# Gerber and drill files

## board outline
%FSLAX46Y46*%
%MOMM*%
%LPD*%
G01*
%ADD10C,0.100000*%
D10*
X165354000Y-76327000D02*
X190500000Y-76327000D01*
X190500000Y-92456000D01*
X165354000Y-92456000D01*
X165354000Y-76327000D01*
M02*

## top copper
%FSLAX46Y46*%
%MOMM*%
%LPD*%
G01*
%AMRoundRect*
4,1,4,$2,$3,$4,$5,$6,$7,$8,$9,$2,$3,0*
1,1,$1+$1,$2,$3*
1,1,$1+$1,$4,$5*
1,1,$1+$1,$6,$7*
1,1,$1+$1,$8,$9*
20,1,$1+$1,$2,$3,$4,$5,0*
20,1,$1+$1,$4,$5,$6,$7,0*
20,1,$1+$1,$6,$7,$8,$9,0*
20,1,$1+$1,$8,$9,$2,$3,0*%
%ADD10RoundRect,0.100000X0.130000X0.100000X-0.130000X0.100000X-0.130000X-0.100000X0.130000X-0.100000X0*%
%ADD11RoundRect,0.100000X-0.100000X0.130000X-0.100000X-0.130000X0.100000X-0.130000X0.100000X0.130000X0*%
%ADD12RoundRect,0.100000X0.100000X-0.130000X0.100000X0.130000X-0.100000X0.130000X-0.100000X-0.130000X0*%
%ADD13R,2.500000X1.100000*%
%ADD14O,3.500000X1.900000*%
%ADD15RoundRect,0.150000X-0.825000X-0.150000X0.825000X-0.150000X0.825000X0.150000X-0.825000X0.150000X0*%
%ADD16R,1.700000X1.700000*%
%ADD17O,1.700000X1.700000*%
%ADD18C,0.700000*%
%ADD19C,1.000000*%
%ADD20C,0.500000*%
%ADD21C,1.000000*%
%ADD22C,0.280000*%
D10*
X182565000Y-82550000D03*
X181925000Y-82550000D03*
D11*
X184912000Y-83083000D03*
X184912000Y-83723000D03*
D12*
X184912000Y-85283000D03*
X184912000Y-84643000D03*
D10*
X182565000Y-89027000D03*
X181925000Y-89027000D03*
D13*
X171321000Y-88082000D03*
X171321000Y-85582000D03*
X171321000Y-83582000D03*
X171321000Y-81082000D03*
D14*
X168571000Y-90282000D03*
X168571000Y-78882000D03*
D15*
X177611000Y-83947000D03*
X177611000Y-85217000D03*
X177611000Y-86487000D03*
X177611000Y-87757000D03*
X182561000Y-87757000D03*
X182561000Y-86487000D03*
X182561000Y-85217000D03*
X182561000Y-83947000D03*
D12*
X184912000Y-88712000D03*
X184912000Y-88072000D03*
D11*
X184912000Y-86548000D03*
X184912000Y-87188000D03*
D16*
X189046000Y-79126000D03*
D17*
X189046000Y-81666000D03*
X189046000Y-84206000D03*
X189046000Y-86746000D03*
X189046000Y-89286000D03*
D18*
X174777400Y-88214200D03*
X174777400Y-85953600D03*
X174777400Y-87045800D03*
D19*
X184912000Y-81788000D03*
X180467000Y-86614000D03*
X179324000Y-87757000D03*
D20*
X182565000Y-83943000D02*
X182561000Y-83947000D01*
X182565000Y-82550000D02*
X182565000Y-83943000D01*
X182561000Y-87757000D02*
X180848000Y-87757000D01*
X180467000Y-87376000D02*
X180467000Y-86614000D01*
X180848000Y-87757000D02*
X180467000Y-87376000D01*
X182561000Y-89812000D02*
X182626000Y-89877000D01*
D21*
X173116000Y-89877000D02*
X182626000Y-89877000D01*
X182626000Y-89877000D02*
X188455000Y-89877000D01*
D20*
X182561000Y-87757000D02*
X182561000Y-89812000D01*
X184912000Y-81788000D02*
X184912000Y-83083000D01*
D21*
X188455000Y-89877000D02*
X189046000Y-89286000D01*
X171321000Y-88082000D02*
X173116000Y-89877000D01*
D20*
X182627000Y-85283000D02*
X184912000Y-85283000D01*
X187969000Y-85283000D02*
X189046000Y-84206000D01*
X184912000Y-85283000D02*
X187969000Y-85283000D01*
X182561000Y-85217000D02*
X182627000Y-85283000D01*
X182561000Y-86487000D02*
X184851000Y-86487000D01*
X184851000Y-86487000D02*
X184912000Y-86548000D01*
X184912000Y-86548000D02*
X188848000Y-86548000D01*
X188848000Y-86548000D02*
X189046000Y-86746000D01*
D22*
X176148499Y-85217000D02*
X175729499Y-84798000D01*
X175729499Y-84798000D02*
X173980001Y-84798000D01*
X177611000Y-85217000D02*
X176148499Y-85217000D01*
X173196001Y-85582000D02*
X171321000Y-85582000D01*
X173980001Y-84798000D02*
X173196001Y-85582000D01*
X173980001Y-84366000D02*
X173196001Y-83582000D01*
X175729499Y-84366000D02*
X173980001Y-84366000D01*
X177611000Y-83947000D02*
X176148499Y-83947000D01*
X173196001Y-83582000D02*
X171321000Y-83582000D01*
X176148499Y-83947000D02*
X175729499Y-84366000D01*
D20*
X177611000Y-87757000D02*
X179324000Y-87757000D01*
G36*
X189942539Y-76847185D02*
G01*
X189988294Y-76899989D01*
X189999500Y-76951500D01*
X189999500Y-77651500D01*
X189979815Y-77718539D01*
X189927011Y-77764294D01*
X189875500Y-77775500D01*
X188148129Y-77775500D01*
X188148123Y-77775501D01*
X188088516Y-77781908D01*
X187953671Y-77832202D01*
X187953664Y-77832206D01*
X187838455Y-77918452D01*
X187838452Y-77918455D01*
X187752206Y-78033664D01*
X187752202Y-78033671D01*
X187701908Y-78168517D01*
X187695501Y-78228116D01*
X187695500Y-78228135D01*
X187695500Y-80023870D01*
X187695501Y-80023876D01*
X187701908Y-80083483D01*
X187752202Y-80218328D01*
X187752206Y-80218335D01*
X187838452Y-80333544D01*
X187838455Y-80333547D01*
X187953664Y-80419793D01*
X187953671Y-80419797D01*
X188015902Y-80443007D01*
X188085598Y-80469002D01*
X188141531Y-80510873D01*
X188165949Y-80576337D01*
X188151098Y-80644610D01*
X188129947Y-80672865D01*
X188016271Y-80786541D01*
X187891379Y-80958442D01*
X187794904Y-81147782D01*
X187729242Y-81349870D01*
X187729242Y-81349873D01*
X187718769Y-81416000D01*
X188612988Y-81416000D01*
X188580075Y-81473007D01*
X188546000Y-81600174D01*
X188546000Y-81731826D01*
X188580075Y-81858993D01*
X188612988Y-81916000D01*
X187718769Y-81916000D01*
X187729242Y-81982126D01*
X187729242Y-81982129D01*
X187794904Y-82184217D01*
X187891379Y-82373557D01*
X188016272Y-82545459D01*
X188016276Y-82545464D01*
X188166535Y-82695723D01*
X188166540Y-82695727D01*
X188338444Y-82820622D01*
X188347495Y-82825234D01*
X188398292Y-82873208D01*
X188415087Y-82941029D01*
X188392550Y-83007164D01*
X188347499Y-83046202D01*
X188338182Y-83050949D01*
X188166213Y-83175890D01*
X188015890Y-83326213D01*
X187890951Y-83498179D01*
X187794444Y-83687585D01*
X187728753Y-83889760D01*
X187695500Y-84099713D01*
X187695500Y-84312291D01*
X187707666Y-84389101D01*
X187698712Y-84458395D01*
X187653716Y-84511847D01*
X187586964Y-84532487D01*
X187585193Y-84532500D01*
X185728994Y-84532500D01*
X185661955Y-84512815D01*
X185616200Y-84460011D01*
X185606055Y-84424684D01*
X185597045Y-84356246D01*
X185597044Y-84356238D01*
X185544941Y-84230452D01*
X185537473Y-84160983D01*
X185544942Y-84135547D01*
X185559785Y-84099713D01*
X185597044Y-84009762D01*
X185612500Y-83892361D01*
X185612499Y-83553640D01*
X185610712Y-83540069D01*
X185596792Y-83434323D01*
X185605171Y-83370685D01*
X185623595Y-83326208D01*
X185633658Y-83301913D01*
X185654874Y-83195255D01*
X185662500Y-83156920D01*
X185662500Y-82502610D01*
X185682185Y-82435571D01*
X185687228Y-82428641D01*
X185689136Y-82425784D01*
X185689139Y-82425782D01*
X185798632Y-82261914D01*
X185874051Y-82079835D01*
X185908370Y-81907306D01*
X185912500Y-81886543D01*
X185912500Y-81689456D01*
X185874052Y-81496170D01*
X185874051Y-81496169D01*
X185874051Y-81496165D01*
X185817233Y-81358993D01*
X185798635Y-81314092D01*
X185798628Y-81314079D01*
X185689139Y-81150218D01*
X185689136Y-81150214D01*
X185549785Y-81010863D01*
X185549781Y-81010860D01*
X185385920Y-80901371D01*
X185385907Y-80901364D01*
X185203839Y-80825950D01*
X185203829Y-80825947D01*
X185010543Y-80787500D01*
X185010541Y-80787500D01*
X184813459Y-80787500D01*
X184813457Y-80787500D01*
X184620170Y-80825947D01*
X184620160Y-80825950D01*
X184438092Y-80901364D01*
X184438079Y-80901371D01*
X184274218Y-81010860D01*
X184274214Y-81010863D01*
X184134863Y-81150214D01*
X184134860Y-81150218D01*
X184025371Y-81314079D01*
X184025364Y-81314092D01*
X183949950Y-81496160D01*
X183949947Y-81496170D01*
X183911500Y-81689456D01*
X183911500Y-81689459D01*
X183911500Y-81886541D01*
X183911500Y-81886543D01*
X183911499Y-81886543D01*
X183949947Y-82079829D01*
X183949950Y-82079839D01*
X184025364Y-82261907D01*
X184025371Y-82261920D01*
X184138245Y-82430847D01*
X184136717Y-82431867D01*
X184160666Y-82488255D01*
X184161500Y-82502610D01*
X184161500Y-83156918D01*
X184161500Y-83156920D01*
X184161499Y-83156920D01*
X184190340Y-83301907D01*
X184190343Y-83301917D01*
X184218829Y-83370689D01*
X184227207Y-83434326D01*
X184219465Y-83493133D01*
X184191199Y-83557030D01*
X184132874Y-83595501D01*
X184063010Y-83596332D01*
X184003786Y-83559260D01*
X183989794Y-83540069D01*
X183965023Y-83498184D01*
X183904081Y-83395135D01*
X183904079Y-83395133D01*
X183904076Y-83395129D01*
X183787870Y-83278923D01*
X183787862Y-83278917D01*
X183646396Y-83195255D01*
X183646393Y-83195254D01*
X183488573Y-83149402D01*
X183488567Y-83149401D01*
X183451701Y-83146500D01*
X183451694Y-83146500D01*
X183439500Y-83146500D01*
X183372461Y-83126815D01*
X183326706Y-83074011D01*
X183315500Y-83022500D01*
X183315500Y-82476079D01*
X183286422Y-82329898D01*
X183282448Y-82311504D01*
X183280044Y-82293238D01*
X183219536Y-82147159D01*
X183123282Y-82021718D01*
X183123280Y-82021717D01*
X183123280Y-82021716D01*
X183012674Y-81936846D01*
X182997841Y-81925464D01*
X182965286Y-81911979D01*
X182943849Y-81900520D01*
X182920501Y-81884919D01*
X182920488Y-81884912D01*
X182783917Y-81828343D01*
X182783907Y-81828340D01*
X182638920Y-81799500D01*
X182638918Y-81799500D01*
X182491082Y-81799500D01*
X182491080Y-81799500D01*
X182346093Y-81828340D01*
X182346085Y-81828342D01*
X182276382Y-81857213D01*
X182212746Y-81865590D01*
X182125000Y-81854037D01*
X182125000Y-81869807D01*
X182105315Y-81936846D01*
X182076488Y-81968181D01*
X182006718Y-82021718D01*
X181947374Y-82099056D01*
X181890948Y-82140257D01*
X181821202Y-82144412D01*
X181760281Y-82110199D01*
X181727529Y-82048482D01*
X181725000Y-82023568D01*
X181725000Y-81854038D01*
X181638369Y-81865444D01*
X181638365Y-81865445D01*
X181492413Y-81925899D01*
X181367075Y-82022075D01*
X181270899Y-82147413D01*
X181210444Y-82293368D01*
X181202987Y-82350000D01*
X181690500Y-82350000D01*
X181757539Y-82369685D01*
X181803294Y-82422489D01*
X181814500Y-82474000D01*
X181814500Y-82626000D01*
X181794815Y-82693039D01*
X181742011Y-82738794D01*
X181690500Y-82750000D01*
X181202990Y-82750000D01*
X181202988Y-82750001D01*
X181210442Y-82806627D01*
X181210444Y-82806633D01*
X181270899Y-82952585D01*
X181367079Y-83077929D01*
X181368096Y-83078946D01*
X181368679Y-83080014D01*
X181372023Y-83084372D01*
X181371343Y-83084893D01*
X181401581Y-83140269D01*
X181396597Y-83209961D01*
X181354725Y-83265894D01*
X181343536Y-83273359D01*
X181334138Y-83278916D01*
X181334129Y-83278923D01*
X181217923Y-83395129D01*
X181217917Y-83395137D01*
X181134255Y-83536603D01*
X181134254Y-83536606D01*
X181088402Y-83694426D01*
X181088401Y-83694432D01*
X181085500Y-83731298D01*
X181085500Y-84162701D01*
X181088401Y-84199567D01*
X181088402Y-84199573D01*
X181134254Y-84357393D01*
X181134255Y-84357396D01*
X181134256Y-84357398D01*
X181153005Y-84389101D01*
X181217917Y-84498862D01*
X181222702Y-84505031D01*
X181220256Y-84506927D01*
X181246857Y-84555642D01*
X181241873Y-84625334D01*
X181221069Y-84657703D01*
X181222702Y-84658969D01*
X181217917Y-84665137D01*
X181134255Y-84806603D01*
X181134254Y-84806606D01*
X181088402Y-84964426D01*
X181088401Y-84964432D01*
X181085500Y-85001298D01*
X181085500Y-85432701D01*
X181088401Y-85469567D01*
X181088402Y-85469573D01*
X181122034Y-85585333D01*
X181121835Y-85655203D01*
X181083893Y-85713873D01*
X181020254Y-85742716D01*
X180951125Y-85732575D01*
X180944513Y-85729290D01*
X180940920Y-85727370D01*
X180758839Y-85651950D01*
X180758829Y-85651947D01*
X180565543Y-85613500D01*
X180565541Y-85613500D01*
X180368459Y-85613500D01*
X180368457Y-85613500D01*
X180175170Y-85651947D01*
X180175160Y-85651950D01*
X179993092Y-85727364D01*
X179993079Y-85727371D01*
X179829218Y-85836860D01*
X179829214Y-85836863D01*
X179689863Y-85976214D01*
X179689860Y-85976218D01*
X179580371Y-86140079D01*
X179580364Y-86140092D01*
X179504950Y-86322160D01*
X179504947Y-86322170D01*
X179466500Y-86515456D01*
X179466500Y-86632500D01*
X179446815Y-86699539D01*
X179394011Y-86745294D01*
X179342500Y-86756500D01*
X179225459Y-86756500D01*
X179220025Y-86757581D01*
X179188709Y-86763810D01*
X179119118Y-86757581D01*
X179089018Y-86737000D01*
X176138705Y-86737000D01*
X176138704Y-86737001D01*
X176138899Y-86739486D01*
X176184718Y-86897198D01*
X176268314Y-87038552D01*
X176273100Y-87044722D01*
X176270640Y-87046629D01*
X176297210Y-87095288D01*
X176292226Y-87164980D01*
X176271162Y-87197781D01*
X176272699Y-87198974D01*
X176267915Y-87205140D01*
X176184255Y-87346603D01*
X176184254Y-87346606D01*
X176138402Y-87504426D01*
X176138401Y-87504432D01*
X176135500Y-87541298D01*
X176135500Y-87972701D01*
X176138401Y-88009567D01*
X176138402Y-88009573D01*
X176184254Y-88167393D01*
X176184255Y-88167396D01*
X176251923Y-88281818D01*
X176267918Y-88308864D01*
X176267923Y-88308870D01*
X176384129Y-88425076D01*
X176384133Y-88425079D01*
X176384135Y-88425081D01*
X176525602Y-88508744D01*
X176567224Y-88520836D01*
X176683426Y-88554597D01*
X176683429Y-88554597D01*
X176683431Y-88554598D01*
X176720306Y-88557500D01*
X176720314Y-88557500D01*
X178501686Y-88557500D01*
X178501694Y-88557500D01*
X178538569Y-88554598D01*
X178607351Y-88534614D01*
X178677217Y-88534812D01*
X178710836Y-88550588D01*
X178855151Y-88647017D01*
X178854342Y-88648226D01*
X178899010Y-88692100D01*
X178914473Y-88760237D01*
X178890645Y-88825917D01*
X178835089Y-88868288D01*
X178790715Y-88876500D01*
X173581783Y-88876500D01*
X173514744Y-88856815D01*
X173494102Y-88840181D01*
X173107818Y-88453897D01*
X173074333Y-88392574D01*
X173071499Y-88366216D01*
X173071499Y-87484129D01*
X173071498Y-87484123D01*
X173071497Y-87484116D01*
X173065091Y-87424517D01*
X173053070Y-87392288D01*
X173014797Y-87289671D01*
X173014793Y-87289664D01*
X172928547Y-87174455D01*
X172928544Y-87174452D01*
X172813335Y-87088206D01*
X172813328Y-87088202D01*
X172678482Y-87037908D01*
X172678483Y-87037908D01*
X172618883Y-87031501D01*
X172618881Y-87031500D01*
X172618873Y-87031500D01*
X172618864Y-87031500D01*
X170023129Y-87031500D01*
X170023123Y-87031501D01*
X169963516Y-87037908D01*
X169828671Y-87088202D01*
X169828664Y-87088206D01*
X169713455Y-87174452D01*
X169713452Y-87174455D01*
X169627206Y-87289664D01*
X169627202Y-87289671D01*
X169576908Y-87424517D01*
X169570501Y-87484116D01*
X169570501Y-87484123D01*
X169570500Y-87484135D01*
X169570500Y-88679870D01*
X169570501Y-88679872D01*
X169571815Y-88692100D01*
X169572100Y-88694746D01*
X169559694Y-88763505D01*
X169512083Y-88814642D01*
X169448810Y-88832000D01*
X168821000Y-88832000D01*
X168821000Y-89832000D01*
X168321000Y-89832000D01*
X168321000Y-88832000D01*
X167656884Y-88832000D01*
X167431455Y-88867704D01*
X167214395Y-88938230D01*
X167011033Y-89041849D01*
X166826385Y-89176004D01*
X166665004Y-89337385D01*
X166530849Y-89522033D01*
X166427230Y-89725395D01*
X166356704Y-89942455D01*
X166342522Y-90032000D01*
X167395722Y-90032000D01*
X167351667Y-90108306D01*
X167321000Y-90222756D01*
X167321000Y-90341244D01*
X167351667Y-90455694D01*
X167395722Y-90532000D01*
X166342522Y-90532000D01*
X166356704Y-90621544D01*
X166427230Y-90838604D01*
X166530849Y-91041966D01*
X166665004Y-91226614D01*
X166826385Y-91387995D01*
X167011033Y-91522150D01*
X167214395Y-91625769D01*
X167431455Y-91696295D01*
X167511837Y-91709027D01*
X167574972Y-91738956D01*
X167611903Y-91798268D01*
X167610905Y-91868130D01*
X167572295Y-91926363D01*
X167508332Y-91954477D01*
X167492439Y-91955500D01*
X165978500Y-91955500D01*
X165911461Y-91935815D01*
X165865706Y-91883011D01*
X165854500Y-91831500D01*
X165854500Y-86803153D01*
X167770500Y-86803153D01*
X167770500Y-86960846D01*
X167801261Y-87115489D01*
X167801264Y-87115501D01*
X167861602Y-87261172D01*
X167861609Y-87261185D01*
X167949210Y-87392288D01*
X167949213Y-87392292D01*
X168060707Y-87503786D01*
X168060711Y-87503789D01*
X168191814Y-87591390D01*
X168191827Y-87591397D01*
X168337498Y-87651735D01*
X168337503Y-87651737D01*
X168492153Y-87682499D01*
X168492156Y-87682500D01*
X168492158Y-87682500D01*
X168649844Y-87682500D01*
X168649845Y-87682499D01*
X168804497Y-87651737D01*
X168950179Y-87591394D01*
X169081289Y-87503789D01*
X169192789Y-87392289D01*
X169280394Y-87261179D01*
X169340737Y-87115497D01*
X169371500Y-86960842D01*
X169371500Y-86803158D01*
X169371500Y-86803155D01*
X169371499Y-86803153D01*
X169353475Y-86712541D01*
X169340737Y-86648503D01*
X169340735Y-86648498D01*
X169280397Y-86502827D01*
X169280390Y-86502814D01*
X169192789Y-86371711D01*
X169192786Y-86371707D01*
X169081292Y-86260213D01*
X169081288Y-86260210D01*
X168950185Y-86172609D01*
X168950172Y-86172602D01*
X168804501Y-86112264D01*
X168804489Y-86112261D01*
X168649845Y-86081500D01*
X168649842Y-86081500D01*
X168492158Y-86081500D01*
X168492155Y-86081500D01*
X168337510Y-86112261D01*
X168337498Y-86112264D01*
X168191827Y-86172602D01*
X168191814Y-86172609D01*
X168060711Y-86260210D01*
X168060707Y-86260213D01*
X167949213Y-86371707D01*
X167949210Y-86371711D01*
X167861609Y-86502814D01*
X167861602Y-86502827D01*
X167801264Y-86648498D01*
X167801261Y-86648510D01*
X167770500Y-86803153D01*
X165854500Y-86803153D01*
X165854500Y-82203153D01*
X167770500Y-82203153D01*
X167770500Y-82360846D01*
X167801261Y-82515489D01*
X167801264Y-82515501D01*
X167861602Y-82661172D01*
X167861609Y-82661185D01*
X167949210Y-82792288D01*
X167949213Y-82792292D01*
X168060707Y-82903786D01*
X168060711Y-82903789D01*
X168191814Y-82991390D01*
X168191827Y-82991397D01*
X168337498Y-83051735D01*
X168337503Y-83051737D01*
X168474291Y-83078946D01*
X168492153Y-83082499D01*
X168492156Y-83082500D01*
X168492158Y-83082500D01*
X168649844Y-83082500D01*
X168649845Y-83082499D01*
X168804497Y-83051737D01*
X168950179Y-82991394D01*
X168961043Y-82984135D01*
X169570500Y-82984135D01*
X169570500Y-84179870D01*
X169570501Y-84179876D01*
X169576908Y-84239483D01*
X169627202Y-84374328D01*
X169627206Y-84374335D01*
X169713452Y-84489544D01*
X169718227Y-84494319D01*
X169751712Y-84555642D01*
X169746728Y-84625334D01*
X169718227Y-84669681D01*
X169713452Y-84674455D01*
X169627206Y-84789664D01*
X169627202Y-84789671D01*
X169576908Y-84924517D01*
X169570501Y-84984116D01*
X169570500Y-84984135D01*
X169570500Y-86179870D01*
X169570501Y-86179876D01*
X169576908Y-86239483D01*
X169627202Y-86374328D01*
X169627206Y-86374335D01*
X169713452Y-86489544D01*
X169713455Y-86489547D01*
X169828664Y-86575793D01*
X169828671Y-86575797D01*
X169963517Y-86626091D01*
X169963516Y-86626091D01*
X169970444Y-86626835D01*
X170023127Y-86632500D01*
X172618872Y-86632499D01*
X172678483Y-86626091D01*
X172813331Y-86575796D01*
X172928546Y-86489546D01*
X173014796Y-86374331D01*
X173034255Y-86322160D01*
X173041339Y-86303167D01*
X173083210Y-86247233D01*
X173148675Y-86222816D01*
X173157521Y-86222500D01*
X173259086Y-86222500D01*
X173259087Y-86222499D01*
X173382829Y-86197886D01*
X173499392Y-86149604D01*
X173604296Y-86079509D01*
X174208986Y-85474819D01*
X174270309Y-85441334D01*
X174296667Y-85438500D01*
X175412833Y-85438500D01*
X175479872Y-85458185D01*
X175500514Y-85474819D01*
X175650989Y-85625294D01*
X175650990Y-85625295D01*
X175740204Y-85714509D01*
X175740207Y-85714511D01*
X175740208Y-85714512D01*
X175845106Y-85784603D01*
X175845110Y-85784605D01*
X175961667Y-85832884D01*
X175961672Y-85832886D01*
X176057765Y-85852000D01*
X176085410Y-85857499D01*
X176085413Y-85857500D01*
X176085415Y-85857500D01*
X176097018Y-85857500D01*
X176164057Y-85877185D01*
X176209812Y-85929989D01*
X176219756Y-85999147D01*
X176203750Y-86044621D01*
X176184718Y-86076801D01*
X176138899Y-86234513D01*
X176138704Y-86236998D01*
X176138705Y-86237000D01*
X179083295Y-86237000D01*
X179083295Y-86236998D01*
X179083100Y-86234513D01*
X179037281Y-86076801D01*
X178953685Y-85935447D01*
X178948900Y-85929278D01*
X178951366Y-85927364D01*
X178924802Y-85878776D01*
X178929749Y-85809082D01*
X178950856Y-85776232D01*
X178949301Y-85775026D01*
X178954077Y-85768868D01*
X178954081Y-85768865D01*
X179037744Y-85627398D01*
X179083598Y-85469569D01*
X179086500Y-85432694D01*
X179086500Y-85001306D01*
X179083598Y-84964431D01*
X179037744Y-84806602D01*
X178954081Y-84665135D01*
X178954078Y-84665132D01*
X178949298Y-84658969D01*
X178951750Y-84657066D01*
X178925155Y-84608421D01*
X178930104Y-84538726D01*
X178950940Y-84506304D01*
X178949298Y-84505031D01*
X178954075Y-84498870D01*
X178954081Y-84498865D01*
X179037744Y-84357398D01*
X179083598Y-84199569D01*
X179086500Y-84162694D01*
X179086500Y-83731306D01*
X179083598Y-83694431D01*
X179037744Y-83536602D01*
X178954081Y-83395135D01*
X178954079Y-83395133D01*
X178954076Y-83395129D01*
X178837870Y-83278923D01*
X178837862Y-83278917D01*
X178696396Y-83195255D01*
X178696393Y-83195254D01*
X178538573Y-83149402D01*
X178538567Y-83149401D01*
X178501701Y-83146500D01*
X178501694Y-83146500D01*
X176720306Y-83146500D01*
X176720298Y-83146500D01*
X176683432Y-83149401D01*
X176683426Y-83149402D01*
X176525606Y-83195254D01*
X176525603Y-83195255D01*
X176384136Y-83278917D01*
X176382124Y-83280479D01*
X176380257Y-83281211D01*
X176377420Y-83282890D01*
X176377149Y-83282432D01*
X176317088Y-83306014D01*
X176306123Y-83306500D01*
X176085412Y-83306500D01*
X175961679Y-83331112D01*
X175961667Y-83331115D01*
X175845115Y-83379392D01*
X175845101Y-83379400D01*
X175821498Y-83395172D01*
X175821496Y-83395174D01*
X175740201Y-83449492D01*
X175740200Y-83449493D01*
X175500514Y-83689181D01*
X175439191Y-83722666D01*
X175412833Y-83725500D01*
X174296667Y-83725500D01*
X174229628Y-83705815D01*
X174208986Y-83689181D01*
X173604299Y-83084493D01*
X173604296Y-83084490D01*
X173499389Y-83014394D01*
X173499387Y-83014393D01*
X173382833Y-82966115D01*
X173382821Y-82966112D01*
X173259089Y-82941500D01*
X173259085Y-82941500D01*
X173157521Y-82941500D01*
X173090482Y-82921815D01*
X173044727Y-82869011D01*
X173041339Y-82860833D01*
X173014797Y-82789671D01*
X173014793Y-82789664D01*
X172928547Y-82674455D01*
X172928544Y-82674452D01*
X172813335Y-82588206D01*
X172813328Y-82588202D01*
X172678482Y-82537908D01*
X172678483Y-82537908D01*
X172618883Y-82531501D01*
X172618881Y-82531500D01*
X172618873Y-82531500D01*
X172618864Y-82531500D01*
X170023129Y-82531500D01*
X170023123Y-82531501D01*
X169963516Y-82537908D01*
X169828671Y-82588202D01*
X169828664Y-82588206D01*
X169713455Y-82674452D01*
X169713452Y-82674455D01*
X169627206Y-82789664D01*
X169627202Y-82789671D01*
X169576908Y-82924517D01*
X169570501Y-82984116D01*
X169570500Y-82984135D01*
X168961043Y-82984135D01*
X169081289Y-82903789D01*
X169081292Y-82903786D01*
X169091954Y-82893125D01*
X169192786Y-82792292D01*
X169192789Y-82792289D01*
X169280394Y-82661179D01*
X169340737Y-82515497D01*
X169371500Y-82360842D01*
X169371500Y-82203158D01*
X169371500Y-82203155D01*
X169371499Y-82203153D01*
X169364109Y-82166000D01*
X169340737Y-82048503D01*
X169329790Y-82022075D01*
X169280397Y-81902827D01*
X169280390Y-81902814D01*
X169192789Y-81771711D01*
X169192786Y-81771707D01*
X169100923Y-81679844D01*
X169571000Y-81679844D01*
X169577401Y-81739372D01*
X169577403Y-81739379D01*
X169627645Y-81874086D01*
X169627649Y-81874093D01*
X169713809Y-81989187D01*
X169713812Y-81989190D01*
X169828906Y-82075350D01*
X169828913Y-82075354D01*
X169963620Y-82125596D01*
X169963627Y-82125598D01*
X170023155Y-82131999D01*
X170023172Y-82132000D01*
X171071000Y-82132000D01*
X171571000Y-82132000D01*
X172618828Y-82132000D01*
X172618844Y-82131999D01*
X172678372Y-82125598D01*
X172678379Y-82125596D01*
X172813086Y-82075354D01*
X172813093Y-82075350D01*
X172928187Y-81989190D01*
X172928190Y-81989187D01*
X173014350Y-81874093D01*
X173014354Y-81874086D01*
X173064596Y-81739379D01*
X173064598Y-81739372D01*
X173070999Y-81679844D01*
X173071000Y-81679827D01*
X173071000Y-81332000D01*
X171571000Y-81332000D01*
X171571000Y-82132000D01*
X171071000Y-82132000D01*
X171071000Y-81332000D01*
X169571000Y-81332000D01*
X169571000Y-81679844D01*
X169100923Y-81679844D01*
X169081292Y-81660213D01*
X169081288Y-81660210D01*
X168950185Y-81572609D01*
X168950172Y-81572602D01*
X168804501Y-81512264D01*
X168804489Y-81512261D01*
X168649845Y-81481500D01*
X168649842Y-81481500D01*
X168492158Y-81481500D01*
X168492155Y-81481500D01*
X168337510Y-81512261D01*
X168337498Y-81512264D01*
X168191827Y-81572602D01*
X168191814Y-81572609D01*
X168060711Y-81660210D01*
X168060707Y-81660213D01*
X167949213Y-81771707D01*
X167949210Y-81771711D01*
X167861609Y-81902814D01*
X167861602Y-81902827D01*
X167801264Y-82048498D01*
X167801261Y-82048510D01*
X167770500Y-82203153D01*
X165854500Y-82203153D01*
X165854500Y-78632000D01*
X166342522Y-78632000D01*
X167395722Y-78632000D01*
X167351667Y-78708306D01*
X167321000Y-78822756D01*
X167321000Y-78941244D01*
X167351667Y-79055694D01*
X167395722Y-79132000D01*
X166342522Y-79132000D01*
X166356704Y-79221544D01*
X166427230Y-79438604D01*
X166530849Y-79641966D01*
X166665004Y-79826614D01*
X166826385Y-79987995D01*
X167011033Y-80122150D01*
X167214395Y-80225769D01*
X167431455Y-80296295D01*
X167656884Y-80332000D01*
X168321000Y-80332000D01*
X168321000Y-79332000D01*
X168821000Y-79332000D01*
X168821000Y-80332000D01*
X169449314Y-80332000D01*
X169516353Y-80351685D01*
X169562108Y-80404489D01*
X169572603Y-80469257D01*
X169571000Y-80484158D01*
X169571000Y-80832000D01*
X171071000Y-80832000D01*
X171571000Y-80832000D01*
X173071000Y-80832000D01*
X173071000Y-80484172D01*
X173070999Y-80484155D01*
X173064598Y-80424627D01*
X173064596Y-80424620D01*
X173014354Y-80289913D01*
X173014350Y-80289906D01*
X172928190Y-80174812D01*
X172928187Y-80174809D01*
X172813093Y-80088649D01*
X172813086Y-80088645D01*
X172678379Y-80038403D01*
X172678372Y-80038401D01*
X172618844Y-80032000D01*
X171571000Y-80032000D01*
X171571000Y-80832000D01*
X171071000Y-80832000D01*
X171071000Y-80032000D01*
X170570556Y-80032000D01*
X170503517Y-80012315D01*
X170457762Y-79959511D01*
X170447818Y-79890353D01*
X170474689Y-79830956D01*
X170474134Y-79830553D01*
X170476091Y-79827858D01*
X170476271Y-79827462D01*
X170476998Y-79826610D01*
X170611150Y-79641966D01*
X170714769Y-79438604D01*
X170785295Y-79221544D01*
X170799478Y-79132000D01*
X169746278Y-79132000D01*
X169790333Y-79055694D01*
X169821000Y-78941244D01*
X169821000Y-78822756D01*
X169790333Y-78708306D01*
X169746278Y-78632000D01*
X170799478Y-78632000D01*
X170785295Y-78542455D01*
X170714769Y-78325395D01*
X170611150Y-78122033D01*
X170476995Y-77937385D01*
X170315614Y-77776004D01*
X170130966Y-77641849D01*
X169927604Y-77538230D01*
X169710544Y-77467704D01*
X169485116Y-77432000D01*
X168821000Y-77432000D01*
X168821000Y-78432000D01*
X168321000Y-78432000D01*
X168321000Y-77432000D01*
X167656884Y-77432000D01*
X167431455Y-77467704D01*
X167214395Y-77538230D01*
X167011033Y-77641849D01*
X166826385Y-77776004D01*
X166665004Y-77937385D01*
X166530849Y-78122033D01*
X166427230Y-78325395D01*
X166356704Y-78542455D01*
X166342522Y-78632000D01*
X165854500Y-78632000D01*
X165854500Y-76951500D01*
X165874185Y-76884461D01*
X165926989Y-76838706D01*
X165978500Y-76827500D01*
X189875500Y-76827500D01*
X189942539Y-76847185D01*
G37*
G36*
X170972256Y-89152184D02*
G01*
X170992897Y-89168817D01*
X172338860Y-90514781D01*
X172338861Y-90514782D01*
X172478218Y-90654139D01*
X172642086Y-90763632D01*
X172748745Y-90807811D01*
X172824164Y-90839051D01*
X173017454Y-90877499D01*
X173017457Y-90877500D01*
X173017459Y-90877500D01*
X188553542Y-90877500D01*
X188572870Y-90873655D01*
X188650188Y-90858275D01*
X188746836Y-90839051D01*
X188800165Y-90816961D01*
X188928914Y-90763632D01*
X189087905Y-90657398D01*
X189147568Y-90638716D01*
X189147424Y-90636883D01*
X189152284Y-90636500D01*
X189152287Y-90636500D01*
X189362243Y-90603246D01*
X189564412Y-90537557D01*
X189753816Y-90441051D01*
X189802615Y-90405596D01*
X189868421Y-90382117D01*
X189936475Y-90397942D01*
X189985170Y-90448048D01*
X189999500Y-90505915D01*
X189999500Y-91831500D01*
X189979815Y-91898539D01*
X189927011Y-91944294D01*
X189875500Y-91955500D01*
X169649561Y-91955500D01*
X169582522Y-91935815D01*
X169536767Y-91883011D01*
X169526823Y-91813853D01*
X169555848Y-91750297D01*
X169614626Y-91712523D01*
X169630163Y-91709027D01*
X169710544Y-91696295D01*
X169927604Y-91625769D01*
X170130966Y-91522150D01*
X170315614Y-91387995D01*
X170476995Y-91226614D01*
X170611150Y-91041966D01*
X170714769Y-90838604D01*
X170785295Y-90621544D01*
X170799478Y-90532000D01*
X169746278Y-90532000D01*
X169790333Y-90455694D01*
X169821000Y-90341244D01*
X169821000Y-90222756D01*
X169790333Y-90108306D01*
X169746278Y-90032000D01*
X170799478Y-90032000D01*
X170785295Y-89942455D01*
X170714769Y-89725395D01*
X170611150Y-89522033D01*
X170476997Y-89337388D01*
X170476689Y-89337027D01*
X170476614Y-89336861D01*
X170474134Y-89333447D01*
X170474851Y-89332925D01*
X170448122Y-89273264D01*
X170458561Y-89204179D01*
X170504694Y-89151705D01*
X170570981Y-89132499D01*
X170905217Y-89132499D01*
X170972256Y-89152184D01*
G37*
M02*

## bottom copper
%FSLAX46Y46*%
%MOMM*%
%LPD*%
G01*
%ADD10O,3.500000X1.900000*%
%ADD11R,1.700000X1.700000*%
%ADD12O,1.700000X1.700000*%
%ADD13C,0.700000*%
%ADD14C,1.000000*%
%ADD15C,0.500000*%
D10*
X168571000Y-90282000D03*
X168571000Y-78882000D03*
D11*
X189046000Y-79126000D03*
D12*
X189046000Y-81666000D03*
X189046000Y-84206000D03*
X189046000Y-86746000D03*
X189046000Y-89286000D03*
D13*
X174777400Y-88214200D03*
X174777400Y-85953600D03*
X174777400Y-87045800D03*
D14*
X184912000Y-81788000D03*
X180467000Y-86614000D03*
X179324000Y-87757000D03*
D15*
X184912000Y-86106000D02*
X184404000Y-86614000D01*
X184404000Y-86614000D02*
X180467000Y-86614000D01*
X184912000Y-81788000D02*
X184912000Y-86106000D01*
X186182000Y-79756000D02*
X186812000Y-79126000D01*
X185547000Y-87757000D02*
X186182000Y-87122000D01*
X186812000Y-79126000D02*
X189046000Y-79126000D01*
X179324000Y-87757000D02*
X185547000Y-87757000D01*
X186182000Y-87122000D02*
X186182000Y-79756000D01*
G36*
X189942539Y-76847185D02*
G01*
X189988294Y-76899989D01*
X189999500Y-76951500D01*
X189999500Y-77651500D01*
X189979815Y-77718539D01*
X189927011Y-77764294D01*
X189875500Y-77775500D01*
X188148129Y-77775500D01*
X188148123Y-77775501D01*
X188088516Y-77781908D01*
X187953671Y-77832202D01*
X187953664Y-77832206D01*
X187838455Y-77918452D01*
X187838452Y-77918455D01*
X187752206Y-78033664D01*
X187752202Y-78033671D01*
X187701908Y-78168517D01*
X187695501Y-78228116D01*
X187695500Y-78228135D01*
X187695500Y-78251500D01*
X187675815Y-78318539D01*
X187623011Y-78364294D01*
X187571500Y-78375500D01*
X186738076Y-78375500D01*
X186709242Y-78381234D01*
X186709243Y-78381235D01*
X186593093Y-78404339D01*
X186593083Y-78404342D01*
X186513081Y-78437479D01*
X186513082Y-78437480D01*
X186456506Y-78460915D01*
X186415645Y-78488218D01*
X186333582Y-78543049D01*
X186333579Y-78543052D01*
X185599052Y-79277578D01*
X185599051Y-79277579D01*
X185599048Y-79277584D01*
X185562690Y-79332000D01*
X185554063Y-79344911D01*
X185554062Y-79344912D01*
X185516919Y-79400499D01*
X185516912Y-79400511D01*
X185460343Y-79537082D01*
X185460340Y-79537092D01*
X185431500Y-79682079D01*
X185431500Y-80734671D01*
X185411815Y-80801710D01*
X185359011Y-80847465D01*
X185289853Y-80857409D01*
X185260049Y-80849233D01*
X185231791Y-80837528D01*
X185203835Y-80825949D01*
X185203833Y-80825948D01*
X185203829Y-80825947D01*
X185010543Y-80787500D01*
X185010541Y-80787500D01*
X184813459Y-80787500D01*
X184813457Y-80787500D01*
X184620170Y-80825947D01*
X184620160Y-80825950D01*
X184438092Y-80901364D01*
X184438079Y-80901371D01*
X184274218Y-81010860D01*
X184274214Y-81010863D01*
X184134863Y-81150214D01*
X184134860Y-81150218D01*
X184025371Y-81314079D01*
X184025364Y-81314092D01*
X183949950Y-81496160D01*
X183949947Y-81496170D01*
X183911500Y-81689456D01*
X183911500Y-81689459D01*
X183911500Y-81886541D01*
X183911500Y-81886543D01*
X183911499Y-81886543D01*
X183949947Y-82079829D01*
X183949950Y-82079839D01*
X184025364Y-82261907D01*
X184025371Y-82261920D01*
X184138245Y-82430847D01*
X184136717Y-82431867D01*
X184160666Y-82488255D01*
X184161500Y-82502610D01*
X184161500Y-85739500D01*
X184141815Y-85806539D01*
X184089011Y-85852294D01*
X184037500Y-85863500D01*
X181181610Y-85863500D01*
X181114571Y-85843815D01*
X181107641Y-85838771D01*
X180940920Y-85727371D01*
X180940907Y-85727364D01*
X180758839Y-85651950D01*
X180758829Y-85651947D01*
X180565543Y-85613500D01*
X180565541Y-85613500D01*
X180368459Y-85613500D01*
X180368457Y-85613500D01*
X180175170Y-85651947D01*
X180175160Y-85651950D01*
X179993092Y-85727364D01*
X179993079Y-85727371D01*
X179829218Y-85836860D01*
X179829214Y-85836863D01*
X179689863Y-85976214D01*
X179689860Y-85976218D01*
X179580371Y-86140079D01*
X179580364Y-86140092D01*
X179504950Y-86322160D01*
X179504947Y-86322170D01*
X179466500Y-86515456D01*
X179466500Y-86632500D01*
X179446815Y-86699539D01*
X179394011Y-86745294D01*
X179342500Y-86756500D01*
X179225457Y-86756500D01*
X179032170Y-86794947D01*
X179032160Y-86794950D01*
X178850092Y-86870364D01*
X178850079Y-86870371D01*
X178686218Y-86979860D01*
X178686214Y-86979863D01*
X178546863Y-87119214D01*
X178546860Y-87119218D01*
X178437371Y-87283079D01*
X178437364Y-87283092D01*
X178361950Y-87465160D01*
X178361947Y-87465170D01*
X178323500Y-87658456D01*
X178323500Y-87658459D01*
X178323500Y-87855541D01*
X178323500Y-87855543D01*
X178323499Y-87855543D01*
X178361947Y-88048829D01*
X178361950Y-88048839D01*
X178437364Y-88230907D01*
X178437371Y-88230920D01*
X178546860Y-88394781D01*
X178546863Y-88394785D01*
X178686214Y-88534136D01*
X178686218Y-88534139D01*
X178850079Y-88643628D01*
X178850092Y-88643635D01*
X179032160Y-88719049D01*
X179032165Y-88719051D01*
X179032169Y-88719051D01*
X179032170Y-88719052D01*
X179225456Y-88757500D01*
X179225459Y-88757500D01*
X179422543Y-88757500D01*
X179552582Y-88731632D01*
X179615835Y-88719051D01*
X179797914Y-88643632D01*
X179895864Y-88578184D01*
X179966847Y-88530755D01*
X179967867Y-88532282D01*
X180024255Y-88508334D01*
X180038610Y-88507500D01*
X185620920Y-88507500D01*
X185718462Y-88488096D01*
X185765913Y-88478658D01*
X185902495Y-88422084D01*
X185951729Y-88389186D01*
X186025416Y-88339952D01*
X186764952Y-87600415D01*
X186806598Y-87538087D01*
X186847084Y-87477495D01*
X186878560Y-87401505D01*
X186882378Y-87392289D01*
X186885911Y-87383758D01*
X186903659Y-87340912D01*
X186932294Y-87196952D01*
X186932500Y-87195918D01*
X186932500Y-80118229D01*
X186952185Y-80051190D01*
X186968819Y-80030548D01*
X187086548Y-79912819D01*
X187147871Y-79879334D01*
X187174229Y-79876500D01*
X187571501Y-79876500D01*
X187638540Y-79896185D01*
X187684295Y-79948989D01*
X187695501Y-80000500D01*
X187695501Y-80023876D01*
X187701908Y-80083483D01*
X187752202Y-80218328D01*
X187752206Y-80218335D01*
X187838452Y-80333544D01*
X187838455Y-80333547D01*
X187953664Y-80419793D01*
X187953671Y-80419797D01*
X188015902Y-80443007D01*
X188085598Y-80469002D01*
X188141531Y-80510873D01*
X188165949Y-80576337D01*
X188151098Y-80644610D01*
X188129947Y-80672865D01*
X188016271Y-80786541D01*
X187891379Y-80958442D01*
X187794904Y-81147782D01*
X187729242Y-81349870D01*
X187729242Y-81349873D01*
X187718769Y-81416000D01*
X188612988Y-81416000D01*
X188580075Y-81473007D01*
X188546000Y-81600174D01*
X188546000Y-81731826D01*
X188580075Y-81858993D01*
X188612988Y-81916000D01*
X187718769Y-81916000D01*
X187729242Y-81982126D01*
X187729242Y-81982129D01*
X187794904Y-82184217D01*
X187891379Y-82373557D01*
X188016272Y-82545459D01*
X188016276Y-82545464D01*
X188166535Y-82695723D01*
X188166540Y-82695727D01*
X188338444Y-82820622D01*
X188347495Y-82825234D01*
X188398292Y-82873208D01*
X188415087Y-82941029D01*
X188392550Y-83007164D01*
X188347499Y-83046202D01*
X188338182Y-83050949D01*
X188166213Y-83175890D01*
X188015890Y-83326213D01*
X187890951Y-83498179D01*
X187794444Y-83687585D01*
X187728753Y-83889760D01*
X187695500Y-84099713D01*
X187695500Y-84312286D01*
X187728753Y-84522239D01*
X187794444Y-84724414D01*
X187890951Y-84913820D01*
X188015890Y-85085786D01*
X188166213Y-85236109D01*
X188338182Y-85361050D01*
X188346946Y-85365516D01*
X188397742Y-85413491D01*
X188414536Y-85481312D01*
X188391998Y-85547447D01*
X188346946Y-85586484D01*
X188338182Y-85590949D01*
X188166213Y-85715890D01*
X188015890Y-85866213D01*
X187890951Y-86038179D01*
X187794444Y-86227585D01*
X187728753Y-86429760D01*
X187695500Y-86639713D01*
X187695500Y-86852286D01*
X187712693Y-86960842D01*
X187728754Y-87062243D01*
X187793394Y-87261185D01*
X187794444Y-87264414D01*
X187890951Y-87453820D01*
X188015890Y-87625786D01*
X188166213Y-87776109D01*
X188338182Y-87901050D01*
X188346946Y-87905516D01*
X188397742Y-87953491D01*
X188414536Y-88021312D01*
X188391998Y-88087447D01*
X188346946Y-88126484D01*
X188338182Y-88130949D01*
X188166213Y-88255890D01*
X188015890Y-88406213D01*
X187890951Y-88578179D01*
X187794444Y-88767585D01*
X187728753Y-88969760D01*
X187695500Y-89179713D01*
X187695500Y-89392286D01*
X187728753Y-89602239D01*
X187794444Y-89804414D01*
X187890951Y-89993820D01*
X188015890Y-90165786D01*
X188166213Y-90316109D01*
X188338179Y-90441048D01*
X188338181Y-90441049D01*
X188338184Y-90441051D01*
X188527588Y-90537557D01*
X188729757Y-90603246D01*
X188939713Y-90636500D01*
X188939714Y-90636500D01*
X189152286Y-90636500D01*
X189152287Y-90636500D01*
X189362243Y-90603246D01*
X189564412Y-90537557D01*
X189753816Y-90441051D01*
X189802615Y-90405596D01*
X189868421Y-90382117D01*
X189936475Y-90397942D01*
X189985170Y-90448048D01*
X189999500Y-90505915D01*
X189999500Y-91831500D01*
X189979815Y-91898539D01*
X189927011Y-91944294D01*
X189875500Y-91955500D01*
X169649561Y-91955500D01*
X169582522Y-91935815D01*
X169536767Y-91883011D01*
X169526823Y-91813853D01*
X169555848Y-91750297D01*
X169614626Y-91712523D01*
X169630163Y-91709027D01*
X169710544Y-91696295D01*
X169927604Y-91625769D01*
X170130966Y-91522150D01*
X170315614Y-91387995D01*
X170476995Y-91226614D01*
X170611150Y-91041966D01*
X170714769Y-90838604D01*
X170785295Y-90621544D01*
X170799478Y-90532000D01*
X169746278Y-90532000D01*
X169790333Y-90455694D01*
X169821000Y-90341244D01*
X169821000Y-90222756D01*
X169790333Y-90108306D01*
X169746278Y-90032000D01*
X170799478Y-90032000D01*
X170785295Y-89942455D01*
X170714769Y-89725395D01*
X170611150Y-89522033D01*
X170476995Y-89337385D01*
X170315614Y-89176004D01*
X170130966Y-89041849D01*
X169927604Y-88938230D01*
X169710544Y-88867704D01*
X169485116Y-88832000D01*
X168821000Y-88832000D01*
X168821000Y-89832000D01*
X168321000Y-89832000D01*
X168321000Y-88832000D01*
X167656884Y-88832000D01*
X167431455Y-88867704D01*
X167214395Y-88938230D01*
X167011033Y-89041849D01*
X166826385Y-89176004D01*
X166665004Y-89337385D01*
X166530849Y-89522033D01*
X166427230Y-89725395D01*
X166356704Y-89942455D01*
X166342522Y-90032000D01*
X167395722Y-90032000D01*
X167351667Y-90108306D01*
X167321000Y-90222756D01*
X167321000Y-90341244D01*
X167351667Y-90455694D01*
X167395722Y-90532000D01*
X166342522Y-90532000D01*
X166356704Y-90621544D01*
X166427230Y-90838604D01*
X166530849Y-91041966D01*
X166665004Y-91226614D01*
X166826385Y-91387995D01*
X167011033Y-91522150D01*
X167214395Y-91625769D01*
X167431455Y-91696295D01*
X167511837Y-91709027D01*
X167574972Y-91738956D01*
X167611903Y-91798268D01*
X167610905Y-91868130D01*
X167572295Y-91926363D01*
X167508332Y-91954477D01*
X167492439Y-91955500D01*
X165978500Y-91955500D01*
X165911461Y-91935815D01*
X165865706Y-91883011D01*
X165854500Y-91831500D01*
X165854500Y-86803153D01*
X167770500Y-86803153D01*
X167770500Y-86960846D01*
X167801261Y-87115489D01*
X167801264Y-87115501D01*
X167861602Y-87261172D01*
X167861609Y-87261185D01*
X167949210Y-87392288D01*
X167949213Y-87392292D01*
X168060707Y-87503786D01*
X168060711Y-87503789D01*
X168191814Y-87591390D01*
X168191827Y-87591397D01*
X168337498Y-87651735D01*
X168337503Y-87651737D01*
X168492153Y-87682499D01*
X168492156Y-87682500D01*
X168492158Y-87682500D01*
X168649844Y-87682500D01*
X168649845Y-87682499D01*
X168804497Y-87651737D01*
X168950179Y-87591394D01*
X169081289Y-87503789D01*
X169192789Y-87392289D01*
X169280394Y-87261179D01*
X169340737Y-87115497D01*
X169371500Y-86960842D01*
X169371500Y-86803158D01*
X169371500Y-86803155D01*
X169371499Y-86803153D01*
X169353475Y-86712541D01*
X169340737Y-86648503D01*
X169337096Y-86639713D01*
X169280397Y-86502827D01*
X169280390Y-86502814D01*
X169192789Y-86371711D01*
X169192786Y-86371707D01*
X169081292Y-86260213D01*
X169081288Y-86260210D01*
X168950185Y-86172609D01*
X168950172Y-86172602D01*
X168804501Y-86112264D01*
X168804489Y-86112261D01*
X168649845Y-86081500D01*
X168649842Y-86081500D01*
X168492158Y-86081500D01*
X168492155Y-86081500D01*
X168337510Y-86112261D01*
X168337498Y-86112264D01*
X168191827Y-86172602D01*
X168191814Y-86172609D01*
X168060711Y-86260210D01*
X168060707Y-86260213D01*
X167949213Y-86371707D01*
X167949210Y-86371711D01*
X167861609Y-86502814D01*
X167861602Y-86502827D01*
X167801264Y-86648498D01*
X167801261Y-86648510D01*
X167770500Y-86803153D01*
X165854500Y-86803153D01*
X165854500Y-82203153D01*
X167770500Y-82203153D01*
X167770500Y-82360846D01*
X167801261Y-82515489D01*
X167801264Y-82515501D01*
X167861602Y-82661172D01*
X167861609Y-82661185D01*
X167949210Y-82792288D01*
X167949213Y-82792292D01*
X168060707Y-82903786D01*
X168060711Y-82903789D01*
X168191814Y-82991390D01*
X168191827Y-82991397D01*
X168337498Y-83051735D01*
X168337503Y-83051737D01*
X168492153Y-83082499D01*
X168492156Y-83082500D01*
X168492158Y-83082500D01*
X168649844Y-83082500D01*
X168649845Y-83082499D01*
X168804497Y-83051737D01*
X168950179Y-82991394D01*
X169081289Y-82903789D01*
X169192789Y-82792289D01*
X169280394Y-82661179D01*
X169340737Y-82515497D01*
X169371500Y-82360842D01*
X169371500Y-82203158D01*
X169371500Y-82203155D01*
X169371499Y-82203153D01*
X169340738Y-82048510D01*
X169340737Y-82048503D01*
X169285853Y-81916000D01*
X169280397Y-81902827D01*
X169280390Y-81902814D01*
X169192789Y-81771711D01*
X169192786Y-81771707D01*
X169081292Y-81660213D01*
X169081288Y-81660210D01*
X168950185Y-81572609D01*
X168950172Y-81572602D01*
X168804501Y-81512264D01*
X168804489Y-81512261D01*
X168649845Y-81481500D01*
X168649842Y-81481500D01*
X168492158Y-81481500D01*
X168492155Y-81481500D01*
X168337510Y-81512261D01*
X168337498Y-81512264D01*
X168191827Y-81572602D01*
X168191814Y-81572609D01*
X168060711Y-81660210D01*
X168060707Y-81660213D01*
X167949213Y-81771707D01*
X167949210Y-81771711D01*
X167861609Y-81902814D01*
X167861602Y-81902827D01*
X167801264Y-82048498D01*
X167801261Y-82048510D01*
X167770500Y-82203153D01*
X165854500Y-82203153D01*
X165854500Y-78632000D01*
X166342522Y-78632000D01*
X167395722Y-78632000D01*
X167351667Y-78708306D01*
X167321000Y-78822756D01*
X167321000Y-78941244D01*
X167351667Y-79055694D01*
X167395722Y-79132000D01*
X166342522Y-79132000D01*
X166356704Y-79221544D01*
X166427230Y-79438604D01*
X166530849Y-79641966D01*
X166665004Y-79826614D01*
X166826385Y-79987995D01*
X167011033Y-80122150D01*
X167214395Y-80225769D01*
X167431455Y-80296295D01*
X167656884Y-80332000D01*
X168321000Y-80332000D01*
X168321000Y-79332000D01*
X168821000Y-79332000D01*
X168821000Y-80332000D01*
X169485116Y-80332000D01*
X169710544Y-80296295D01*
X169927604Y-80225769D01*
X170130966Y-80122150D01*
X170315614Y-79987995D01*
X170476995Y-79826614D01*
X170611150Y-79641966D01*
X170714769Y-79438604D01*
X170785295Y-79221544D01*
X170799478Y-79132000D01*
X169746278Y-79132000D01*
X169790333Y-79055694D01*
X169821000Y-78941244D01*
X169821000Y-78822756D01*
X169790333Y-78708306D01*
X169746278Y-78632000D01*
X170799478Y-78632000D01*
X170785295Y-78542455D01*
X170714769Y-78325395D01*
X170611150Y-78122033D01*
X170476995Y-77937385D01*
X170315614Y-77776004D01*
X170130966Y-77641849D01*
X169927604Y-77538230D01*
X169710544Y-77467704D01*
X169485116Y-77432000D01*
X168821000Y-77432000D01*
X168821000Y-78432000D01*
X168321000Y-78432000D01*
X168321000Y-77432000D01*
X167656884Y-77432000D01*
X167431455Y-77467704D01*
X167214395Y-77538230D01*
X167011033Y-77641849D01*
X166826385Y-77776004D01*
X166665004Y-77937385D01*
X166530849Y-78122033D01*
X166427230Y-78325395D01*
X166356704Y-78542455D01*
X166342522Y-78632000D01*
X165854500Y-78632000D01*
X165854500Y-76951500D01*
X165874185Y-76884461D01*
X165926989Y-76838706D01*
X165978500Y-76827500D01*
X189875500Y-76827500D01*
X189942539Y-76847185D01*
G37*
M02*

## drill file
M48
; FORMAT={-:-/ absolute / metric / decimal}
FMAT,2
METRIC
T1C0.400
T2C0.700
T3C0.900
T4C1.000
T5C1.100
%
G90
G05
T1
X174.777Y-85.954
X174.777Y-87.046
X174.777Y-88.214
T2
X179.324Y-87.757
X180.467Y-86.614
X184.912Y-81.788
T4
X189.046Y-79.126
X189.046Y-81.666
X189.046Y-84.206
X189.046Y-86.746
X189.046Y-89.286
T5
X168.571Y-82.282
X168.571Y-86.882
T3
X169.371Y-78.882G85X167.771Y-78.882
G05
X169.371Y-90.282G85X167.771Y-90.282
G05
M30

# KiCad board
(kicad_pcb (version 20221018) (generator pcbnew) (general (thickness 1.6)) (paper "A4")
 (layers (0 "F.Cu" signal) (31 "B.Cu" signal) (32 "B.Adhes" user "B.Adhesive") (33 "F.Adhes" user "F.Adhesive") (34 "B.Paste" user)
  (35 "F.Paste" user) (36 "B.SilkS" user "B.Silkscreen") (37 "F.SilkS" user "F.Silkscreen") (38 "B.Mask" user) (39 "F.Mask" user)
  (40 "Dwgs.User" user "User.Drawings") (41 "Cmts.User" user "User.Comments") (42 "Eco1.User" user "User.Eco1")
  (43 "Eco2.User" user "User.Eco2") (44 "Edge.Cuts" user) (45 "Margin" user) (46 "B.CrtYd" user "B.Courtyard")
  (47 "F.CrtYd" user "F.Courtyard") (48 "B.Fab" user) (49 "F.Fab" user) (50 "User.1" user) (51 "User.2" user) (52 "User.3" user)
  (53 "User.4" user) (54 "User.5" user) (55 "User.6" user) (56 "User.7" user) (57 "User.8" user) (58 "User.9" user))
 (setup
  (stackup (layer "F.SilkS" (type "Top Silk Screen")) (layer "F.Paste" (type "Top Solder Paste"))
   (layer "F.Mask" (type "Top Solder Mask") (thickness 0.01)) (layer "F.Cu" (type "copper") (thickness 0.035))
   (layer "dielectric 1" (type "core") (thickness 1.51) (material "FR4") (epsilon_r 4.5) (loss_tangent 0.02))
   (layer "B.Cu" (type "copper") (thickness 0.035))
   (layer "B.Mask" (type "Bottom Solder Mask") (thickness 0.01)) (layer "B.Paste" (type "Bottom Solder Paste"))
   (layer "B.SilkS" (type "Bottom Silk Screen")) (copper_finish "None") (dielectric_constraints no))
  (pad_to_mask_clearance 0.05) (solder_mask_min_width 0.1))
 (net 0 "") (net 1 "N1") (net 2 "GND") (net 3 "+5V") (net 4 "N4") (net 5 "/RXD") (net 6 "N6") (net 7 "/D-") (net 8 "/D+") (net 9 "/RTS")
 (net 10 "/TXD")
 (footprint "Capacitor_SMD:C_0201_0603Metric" (layer "F.Cu") (at 182.245 82.55 180)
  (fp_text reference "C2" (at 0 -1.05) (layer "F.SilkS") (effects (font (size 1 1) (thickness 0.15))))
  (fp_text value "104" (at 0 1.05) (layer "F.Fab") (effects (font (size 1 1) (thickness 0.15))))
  (pad "" smd roundrect (at -0.345 0 180) (size 0.318 0.36) (layers "F.Paste") (roundrect_rratio 0.25))
  (pad "" smd roundrect (at 0.345 0 180) (size 0.318 0.36) (layers "F.Paste") (roundrect_rratio 0.25))
  (pad "1" smd roundrect (at -0.32 0 180) (size 0.46 0.4) (layers "F.Cu" "F.Mask") (roundrect_rratio 0.25) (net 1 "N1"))
  (pad "2" smd roundrect (at 0.32 0 180) (size 0.46 0.4) (layers "F.Cu" "F.Mask") (roundrect_rratio 0.25) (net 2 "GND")))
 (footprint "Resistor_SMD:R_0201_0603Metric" (layer "F.Cu") (at 184.912 83.403 -90)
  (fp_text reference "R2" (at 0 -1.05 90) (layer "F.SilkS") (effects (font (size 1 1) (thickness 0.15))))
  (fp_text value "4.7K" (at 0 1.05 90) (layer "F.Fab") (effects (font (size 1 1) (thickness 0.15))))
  (pad "" smd roundrect (at -0.345 0 270) (size 0.318 0.36) (layers "F.Paste") (roundrect_rratio 0.25))
  (pad "" smd roundrect (at 0.345 0 270) (size 0.318 0.36) (layers "F.Paste") (roundrect_rratio 0.25))
  (pad "1" smd roundrect (at -0.32 0 270) (size 0.46 0.4) (layers "F.Cu" "F.Mask") (roundrect_rratio 0.25) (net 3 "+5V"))
  (pad "2" smd roundrect (at 0.32 0 270) (size 0.46 0.4) (layers "F.Cu" "F.Mask") (roundrect_rratio 0.25) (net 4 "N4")))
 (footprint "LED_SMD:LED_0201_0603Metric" (layer "F.Cu") (at 184.912 84.963 90)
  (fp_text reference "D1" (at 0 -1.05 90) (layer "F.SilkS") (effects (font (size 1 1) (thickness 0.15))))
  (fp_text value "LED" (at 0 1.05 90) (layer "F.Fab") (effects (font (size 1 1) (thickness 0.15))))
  (pad "" smd roundrect (at -0.345 0 90) (size 0.318 0.36) (layers "F.Paste") (roundrect_rratio 0.25))
  (pad "" smd roundrect (at 0.345 0 90) (size 0.318 0.36) (layers "F.Paste") (roundrect_rratio 0.25))
  (pad "1" smd roundrect (at -0.32 0 90) (size 0.46 0.4) (layers "F.Cu" "F.Mask") (roundrect_rratio 0.25) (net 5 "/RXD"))
  (pad "2" smd roundrect (at 0.32 0 90) (size 0.46 0.4) (layers "F.Cu" "F.Mask") (roundrect_rratio 0.25) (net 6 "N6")))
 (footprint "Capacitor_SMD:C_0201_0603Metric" (layer "F.Cu") (at 182.245 89.027 180)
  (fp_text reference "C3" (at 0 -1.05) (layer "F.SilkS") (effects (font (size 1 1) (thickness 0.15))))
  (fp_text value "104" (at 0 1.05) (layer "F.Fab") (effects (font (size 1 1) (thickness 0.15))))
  (pad "" smd roundrect (at -0.345 0 180) (size 0.318 0.36) (layers "F.Paste") (roundrect_rratio 0.25))
  (pad "" smd roundrect (at 0.345 0 180) (size 0.318 0.36) (layers "F.Paste") (roundrect_rratio 0.25))
  (pad "1" smd roundrect (at -0.32 0 180) (size 0.46 0.4) (layers "F.Cu" "F.Mask") (roundrect_rratio 0.25) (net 3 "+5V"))
  (pad "2" smd roundrect (at 0.32 0 180) (size 0.46 0.4) (layers "F.Cu" "F.Mask") (roundrect_rratio 0.25) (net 2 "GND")))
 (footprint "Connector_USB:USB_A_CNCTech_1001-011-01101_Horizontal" (layer "F.Cu") (at 161.671 84.582 180)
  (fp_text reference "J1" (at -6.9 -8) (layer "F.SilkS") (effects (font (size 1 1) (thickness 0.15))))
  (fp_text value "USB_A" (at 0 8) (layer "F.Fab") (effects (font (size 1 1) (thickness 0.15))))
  (pad "" np_thru_hole circle (at -6.9 -2.3 180) (size 1.1 1.1) (drill 1.1) (layers "*.Cu" "*.Mask"))
  (pad "" np_thru_hole circle (at -6.9 2.3 180) (size 1.1 1.1) (drill 1.1) (layers "*.Cu" "*.Mask"))
  (pad "1" smd rect (at -9.65 -3.5 180) (size 2.5 1.1) (layers "F.Cu" "F.Paste" "F.Mask") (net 3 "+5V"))
  (pad "2" smd rect (at -9.65 -1 180) (size 2.5 1.1) (layers "F.Cu" "F.Paste" "F.Mask") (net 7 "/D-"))
  (pad "3" smd rect (at -9.65 1 180) (size 2.5 1.1) (layers "F.Cu" "F.Paste" "F.Mask") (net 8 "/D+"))
  (pad "4" smd rect (at -9.65 3.5 180) (size 2.5 1.1) (layers "F.Cu" "F.Paste" "F.Mask") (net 2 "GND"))
  (pad "5" thru_hole oval (at -6.9 -5.7 180) (size 3.5 1.9) (drill oval 2.5 0.9) (layers "*.Cu" "*.Mask") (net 2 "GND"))
  (pad "5" thru_hole oval (at -6.9 5.7 180) (size 3.5 1.9) (drill oval 2.5 0.9) (layers "*.Cu" "*.Mask") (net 2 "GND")))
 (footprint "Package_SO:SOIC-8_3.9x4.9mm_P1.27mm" (layer "F.Cu") (at 180.086 85.852)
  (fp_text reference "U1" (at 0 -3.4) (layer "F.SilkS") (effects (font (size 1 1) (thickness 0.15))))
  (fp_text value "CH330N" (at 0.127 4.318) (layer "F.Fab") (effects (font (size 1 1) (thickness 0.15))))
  (pad "1" smd roundrect (at -2.475 -1.905) (size 1.95 0.6) (layers "F.Cu" "F.Paste" "F.Mask") (roundrect_rratio 0.25) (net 8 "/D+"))
  (pad "2" smd roundrect (at -2.475 -0.635) (size 1.95 0.6) (layers "F.Cu" "F.Paste" "F.Mask") (roundrect_rratio 0.25) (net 7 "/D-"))
  (pad "3" smd roundrect (at -2.475 0.635) (size 1.95 0.6) (layers "F.Cu" "F.Paste" "F.Mask") (roundrect_rratio 0.25) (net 2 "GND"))
  (pad "4" smd roundrect (at -2.475 1.905) (size 1.95 0.6) (layers "F.Cu" "F.Paste" "F.Mask") (roundrect_rratio 0.25) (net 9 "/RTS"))
  (pad "5" smd roundrect (at 2.475 1.905) (size 1.95 0.6) (layers "F.Cu" "F.Paste" "F.Mask") (roundrect_rratio 0.25) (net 3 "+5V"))
  (pad "6" smd roundrect (at 2.475 0.635) (size 1.95 0.6) (layers "F.Cu" "F.Paste" "F.Mask") (roundrect_rratio 0.25) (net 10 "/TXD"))
  (pad "7" smd roundrect (at 2.475 -0.635) (size 1.95 0.6) (layers "F.Cu" "F.Paste" "F.Mask") (roundrect_rratio 0.25) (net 5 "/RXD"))
  (pad "8" smd roundrect (at 2.475 -1.905) (size 1.95 0.6) (layers "F.Cu" "F.Paste" "F.Mask") (roundrect_rratio 0.25) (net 1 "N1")))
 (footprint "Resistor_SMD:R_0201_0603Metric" (layer "F.Cu") (at 184.912 88.392 90)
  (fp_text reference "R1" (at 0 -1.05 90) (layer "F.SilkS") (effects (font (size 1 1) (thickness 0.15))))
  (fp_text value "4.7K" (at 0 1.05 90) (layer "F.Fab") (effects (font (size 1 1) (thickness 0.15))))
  (pad "" smd roundrect (at -0.345 0 90) (size 0.318 0.36) (layers "F.Paste") (roundrect_rratio 0.25))
  (pad "" smd roundrect (at 0.345 0 90) (size 0.318 0.36) (layers "F.Paste") (roundrect_rratio 0.25))
  (pad "1" smd roundrect (at -0.32 0 90) (size 0.46 0.4) (layers "F.Cu" "F.Mask") (roundrect_rratio 0.25) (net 3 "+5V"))
  (pad "2" smd roundrect (at 0.32 0 90) (size 0.46 0.4) (layers "F.Cu" "F.Mask") (roundrect_rratio 0.25) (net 6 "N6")))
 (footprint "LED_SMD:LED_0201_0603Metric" (layer "F.Cu") (at 184.912 86.868 -90)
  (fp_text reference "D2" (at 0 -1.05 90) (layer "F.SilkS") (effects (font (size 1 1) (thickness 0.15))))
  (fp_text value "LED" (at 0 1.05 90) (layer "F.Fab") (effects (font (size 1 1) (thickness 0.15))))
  (pad "" smd roundrect (at -0.345 0 270) (size 0.318 0.36) (layers "F.Paste") (roundrect_rratio 0.25))
  (pad "" smd roundrect (at 0.345 0 270) (size 0.318 0.36) (layers "F.Paste") (roundrect_rratio 0.25))
  (pad "1" smd roundrect (at -0.32 0 270) (size 0.46 0.4) (layers "F.Cu" "F.Mask") (roundrect_rratio 0.25) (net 10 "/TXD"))
  (pad "2" smd roundrect (at 0.32 0 270) (size 0.46 0.4) (layers "F.Cu" "F.Mask") (roundrect_rratio 0.25) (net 4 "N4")))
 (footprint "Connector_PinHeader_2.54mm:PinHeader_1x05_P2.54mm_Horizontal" (layer "F.Cu") (at 189.046 79.126)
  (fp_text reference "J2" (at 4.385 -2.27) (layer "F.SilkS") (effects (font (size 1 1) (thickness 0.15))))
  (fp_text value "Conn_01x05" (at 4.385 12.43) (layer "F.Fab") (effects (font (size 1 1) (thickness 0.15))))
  (pad "1" thru_hole rect (at 0 0) (size 1.7 1.7) (drill 1) (layers "*.Cu" "*.Mask") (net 9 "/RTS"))
  (pad "2" thru_hole oval (at 0 2.54) (size 1.7 1.7) (drill 1) (layers "*.Cu" "*.Mask") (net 2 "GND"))
  (pad "3" thru_hole oval (at 0 5.08) (size 1.7 1.7) (drill 1) (layers "*.Cu" "*.Mask") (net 5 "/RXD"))
  (pad "4" thru_hole oval (at 0 7.62) (size 1.7 1.7) (drill 1) (layers "*.Cu" "*.Mask") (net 10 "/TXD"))
  (pad "5" thru_hole oval (at 0 10.16) (size 1.7 1.7) (drill 1) (layers "*.Cu" "*.Mask") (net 3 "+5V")))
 (gr_rect (start 165.354 76.327) (end 190.5 92.456) (stroke (width 0.1) (type default)) (fill none) (layer "Edge.Cuts"))
 (segment (start 182.565 83.943) (end 182.561 83.947) (width 0.5) (layer "F.Cu") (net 1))
 (segment (start 182.565 82.55) (end 182.565 83.943) (width 0.5) (layer "F.Cu") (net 1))
 (via (at 174.7774 88.2142) (size 0.7) (drill 0.4) (layers "F.Cu" "B.Cu") (free) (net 2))
 (via (at 174.7774 85.9536) (size 0.7) (drill 0.4) (layers "F.Cu" "B.Cu") (free) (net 2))
 (via (at 174.7774 87.0458) (size 0.7) (drill 0.4) (layers "F.Cu" "B.Cu") (free) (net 2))
 (segment (start 182.561 87.757) (end 180.848 87.757) (width 0.5) (layer "F.Cu") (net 3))
 (segment (start 180.467 87.376) (end 180.467 86.614) (width 0.5) (layer "F.Cu") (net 3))
 (segment (start 180.848 87.757) (end 180.467 87.376) (width 0.5) (layer "F.Cu") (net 3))
 (segment (start 182.561 89.812) (end 182.626 89.877) (width 0.5) (layer "F.Cu") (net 3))
 (segment (start 173.116 89.877) (end 182.626 89.877) (width 1) (layer "F.Cu") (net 3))
 (segment (start 182.626 89.877) (end 188.455 89.877) (width 1) (layer "F.Cu") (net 3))
 (segment (start 182.561 87.757) (end 182.561 89.812) (width 0.5) (layer "F.Cu") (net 3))
 (segment (start 184.912 81.788) (end 184.912 83.083) (width 0.5) (layer "F.Cu") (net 3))
 (segment (start 188.455 89.877) (end 189.046 89.286) (width 1) (layer "F.Cu") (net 3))
 (segment (start 171.321 88.082) (end 173.116 89.877) (width 1) (layer "F.Cu") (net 3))
 (via (at 184.912 81.788) (size 1) (drill 0.7) (layers "F.Cu" "B.Cu") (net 3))
 (via (at 180.467 86.614) (size 1) (drill 0.7) (layers "F.Cu" "B.Cu") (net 3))
 (segment (start 184.912 86.106) (end 184.404 86.614) (width 0.5) (layer "B.Cu") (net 3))
 (segment (start 184.404 86.614) (end 180.467 86.614) (width 0.5) (layer "B.Cu") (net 3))
 (segment (start 184.912 81.788) (end 184.912 86.106) (width 0.5) (layer "B.Cu") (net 3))
 (segment (start 182.627 85.283) (end 184.912 85.283) (width 0.5) (layer "F.Cu") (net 5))
 (segment (start 187.969 85.283) (end 189.046 84.206) (width 0.5) (layer "F.Cu") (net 5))
 (segment (start 184.912 85.283) (end 187.969 85.283) (width 0.5) (layer "F.Cu") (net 5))
 (segment (start 182.561 85.217) (end 182.627 85.283) (width 0.5) (layer "F.Cu") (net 5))
 (segment (start 182.561 86.487) (end 184.851 86.487) (width 0.5) (layer "F.Cu") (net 10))
 (segment (start 184.851 86.487) (end 184.912 86.548) (width 0.5) (layer "F.Cu") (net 10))
 (segment (start 184.912 86.548) (end 188.848 86.548) (width 0.5) (layer "F.Cu") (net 10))
 (segment (start 188.848 86.548) (end 189.046 86.746) (width 0.5) (layer "F.Cu") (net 10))
 (segment (start 176.148499 85.217) (end 175.729499 84.798) (width 0.28) (layer "F.Cu") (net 7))
 (segment (start 175.729499 84.798) (end 173.980001 84.798) (width 0.28) (layer "F.Cu") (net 7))
 (segment (start 177.611 85.217) (end 176.148499 85.217) (width 0.28) (layer "F.Cu") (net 7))
 (segment (start 173.196001 85.582) (end 171.321 85.582) (width 0.28) (layer "F.Cu") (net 7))
 (segment (start 173.980001 84.798) (end 173.196001 85.582) (width 0.28) (layer "F.Cu") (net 7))
 (segment (start 173.980001 84.366) (end 173.196001 83.582) (width 0.28) (layer "F.Cu") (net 8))
 (segment (start 175.729499 84.366) (end 173.980001 84.366) (width 0.28) (layer "F.Cu") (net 8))
 (segment (start 177.611 83.947) (end 176.148499 83.947) (width 0.28) (layer "F.Cu") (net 8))
 (segment (start 173.196001 83.582) (end 171.321 83.582) (width 0.28) (layer "F.Cu") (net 8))
 (segment (start 176.148499 83.947) (end 175.729499 84.366) (width 0.28) (layer "F.Cu") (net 8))
 (segment (start 177.611 87.757) (end 179.324 87.757) (width 0.5) (layer "F.Cu") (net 9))
 (via (at 179.324 87.757) (size 1) (drill 0.7) (layers "F.Cu" "B.Cu") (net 9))
 (segment (start 186.182 79.756) (end 186.812 79.126) (width 0.5) (layer "B.Cu") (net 9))
 (segment (start 185.547 87.757) (end 186.182 87.122) (width 0.5) (layer "B.Cu") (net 9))
 (segment (start 186.812 79.126) (end 189.046 79.126) (width 0.5) (layer "B.Cu") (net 9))
 (segment (start 179.324 87.757) (end 185.547 87.757) (width 0.5) (layer "B.Cu") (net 9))
 (segment (start 186.182 87.122) (end 186.182 79.756) (width 0.5) (layer "B.Cu") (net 9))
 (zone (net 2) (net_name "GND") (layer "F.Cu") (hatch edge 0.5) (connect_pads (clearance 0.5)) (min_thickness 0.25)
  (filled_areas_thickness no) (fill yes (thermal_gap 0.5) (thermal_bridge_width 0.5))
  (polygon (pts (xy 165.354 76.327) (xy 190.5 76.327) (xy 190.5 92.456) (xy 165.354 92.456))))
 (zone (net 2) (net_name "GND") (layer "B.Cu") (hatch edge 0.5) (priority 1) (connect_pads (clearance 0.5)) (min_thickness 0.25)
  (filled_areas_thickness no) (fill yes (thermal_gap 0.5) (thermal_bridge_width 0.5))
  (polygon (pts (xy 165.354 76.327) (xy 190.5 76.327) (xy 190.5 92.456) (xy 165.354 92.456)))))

